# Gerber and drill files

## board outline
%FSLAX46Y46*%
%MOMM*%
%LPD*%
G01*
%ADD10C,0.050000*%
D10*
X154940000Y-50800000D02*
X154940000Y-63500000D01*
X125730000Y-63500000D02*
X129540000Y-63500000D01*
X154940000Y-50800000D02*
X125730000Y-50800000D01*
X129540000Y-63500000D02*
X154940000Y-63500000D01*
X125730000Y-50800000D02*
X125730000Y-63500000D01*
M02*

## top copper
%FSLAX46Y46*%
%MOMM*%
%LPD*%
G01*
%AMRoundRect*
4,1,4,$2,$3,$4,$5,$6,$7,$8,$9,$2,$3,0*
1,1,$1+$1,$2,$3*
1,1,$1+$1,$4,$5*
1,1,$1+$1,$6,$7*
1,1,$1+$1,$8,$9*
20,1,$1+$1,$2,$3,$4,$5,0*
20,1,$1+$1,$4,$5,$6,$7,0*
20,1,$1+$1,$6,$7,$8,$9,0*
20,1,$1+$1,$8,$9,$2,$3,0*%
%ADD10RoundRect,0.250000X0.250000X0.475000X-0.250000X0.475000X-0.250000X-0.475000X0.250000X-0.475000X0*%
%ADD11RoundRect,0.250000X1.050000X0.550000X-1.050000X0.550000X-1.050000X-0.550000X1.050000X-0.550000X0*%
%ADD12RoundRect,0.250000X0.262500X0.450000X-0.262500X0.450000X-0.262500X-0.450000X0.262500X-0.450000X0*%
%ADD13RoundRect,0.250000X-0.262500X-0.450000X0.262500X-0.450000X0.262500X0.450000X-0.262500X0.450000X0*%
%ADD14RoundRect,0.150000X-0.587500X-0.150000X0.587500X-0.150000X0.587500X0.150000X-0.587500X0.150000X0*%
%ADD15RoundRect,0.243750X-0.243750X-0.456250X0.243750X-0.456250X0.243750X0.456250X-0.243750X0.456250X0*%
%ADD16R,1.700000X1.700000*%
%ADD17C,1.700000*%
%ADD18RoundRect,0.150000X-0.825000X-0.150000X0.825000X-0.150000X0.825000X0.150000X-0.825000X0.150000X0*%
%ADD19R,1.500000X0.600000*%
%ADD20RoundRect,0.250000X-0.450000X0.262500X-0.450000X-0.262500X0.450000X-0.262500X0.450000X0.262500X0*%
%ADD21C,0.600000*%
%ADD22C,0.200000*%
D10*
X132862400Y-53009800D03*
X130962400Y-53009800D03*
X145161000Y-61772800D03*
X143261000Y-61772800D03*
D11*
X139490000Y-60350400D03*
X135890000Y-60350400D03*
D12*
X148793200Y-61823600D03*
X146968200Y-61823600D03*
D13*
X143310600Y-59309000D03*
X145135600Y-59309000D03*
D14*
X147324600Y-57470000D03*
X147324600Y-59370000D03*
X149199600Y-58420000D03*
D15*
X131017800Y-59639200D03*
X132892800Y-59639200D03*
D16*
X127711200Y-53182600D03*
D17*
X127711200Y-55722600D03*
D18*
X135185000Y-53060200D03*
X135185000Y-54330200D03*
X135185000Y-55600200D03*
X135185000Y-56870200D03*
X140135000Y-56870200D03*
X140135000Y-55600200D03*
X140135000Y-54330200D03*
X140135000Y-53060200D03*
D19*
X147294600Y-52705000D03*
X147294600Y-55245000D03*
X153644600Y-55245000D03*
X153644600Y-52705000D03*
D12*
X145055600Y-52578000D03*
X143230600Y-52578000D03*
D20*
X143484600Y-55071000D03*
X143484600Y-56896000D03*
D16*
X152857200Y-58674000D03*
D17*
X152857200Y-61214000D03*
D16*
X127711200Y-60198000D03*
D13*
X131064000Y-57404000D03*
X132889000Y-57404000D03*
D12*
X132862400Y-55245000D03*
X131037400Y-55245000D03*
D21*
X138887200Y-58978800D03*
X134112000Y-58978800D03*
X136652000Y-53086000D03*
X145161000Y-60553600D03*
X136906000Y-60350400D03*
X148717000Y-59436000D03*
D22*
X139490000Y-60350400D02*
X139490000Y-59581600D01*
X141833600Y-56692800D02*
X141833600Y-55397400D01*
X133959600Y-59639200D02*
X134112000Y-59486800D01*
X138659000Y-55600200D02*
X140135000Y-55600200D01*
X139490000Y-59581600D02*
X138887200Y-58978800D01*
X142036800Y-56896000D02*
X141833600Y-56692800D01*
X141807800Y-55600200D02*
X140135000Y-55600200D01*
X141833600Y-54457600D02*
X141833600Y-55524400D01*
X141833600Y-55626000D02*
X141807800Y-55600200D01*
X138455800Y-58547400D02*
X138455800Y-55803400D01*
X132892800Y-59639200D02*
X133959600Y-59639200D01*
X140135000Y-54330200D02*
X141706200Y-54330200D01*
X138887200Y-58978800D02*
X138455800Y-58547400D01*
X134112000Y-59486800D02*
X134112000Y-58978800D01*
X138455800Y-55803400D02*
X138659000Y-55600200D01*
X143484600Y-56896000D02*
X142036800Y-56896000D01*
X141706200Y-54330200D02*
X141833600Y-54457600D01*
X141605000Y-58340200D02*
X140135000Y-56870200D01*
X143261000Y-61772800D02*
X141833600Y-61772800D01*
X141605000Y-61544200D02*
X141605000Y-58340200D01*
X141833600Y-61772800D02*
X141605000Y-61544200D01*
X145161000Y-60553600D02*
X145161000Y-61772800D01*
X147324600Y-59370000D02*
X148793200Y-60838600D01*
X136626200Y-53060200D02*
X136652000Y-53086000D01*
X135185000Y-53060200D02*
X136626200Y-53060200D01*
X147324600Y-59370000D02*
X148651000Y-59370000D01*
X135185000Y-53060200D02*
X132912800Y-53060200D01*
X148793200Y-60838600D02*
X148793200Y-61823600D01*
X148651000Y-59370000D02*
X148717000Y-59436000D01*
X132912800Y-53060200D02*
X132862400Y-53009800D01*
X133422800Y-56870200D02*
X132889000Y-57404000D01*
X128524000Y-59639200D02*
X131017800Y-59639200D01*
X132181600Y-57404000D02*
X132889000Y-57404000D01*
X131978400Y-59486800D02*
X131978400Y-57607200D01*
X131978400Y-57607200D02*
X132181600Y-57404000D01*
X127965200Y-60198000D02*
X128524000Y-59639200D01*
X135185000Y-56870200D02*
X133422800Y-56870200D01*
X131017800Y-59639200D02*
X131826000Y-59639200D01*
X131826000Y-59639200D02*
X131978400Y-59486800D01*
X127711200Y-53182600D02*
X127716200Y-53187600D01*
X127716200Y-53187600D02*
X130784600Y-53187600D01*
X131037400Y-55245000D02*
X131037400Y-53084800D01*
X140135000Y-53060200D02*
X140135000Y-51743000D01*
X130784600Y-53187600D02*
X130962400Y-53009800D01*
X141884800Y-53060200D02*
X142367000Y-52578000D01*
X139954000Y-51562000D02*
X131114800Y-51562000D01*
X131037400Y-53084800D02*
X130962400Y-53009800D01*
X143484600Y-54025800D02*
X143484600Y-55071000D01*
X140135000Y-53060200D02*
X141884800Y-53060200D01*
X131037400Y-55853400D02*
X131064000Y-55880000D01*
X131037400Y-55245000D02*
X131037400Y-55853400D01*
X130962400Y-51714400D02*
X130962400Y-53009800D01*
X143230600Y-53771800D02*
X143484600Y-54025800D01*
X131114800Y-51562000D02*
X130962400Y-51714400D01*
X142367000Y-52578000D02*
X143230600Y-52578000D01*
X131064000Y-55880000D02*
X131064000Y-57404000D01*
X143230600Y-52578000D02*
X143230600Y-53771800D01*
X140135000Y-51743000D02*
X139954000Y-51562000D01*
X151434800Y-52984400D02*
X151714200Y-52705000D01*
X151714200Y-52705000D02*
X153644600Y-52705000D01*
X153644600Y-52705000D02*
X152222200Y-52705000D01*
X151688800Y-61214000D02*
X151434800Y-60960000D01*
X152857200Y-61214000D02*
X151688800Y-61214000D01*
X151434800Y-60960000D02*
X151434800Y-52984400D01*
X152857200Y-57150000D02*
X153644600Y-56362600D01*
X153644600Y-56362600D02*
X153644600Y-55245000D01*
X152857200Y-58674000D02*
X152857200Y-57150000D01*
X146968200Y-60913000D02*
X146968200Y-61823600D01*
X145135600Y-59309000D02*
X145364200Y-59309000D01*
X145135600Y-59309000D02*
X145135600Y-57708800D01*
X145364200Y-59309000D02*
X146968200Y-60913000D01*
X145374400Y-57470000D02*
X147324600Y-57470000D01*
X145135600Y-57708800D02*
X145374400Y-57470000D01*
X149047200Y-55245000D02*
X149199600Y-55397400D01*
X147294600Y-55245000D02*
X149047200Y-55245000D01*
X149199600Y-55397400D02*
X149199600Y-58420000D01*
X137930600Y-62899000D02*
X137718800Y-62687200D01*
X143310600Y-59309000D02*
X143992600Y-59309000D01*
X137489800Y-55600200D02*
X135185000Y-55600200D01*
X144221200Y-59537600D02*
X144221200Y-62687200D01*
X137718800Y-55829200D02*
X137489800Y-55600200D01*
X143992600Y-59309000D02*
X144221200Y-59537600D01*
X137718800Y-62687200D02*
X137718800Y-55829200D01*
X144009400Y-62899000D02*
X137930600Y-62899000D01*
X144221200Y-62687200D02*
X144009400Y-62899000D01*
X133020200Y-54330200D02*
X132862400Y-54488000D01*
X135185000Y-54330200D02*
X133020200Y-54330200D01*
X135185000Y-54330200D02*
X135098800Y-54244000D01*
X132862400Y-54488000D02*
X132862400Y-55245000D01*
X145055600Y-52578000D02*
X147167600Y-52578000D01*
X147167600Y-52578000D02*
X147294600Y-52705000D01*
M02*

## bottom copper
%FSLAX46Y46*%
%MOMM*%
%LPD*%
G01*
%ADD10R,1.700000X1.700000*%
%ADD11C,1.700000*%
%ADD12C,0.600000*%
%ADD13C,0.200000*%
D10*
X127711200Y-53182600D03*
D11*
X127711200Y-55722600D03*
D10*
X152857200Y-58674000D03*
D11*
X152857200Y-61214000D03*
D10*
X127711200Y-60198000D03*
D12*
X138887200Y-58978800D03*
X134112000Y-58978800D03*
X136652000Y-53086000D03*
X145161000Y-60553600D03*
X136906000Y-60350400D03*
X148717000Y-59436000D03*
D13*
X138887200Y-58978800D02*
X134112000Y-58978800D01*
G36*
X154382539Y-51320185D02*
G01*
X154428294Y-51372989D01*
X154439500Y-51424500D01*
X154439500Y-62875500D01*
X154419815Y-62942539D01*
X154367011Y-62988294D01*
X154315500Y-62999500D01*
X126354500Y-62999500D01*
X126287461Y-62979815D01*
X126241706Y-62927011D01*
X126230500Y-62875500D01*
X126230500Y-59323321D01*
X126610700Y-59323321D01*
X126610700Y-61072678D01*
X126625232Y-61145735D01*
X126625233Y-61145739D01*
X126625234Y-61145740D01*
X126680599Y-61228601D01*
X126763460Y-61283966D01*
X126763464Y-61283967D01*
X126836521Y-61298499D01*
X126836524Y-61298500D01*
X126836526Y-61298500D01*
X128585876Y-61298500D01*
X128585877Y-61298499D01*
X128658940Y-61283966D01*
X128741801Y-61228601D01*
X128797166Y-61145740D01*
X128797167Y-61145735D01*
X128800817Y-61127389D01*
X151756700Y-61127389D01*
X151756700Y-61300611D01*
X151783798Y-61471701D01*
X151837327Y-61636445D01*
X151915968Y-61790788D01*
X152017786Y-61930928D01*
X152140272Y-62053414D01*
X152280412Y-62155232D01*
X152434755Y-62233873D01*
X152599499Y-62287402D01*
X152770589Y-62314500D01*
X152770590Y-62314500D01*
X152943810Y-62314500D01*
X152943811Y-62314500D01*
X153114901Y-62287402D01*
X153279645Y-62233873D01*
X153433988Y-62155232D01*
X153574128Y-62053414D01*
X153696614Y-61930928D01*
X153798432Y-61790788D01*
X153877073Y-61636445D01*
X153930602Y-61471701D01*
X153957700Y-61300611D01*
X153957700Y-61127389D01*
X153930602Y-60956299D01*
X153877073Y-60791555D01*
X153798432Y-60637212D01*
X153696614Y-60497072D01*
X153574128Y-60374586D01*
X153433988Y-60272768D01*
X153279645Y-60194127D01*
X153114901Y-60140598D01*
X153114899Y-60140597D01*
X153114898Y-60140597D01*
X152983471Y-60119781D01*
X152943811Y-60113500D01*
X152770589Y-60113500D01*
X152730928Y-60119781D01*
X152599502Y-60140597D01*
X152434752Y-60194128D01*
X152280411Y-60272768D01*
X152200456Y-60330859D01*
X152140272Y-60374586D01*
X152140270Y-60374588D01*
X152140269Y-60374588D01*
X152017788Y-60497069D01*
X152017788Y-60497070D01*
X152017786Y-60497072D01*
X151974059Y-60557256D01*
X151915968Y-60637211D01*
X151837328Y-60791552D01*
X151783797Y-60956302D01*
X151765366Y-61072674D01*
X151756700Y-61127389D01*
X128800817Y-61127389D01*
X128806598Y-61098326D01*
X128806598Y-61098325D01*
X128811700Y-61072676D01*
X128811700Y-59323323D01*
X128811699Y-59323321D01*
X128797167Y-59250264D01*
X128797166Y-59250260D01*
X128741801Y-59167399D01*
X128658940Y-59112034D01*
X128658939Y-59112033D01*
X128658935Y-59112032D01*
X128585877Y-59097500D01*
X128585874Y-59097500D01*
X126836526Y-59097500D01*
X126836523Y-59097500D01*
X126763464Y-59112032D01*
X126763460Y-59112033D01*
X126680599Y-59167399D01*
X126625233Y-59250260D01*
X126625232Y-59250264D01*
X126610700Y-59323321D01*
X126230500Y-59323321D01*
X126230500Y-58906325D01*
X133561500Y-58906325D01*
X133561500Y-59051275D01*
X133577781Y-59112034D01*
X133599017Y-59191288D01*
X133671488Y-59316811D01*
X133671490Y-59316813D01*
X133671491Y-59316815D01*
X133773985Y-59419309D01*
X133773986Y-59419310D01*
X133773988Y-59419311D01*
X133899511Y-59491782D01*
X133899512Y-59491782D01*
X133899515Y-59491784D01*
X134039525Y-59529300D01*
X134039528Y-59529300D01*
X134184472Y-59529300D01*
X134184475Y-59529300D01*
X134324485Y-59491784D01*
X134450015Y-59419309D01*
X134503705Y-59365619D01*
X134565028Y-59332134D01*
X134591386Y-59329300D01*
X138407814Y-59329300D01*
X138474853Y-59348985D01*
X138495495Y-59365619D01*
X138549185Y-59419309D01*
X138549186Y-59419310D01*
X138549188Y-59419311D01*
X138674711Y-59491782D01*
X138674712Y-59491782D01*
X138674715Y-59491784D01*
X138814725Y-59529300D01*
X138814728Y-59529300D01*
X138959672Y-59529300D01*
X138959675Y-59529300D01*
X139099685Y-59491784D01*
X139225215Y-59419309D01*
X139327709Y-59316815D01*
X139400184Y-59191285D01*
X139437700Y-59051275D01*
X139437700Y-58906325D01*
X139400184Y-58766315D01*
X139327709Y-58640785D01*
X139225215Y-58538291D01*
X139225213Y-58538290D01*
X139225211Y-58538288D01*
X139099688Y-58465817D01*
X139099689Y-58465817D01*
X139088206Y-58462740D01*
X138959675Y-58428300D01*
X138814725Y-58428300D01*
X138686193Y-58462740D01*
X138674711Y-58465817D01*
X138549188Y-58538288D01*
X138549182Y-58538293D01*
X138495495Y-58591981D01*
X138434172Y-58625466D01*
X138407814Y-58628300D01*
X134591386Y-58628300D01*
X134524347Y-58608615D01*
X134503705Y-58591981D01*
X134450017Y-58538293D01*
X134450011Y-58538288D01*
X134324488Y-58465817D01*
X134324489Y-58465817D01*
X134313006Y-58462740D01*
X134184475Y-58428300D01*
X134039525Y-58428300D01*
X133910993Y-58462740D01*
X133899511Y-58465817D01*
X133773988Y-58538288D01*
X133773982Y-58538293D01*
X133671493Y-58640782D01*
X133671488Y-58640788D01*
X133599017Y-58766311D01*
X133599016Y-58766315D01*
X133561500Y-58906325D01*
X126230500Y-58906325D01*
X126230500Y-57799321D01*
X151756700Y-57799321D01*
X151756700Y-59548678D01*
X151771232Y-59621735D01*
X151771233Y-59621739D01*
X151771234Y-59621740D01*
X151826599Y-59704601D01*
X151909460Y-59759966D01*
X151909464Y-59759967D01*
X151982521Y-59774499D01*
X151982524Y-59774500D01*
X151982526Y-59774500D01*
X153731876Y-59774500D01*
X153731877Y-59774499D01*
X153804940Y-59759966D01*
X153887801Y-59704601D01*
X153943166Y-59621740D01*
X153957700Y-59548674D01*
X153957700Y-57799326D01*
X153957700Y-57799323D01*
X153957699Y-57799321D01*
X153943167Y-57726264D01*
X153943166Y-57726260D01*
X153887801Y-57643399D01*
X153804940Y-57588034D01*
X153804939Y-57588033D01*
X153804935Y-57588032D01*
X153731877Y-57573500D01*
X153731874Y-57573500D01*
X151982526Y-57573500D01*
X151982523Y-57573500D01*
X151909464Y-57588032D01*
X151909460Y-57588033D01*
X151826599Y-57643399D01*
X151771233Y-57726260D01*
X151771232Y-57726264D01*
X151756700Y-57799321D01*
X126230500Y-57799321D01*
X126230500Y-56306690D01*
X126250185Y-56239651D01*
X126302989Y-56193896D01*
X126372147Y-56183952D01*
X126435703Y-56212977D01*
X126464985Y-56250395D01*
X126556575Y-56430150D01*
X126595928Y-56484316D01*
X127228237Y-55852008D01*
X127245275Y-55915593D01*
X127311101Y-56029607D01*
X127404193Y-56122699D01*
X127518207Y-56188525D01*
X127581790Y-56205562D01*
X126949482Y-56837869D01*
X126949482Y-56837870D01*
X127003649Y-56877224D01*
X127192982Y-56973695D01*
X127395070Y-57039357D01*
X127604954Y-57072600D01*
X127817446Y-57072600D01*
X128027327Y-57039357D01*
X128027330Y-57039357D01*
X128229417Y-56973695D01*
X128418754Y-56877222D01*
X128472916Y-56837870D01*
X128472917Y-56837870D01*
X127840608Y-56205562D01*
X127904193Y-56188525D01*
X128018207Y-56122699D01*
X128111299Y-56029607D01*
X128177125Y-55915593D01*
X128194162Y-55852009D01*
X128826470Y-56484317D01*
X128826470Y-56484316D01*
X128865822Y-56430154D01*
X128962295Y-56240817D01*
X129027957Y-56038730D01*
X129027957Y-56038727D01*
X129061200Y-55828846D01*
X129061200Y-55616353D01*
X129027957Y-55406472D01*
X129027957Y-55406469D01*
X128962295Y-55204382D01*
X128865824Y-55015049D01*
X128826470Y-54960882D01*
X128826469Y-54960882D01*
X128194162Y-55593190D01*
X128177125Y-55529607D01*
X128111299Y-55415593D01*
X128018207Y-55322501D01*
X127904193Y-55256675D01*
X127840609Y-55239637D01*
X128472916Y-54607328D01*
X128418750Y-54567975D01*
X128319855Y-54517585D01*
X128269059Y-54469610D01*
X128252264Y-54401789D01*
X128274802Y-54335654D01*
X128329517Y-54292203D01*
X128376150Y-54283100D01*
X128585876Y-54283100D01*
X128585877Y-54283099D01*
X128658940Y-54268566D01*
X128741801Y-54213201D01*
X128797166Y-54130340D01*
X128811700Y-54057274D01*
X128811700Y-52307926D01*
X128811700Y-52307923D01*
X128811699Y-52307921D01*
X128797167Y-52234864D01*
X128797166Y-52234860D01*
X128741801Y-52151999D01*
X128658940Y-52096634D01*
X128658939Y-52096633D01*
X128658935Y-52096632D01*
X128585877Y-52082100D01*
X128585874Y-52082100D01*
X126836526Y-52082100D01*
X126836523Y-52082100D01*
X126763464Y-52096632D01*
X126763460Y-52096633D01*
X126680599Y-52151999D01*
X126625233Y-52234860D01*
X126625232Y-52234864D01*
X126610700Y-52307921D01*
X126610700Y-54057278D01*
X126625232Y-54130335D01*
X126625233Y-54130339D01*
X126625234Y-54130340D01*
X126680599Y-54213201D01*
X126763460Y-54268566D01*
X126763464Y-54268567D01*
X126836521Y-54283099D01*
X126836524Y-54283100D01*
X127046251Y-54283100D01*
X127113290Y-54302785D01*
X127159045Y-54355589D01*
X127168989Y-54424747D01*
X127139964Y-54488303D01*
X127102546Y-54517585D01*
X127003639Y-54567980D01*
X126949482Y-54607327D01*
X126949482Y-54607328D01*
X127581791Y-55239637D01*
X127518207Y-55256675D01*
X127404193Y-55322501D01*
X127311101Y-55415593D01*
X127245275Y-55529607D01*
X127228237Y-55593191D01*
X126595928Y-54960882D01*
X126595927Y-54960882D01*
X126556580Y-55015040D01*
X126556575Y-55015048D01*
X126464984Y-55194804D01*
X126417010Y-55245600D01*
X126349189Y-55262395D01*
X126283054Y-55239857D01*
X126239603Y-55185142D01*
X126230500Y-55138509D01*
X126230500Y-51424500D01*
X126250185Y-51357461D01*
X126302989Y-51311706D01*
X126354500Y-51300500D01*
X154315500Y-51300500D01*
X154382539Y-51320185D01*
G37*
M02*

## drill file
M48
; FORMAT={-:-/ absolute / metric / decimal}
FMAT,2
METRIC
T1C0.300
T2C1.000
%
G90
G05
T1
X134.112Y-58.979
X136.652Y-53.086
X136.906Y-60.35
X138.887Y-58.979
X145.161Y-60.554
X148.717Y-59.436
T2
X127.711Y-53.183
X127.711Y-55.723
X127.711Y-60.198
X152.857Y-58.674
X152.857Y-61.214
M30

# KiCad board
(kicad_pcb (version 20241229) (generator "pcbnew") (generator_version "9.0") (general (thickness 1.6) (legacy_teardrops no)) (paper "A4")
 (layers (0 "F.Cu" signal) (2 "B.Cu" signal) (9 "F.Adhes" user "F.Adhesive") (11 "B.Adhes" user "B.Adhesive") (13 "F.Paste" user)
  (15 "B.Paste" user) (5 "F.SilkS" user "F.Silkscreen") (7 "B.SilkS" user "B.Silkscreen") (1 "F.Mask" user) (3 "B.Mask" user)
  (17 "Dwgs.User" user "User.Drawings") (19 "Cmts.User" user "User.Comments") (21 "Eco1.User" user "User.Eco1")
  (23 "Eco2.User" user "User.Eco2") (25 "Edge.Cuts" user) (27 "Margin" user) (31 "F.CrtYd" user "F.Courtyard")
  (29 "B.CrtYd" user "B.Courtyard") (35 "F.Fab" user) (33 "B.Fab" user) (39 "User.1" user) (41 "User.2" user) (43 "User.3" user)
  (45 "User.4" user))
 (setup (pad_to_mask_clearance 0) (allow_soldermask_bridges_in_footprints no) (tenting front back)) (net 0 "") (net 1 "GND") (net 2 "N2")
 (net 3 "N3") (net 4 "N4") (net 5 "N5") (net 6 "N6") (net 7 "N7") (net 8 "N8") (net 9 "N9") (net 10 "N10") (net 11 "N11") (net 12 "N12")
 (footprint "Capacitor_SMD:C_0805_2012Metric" (layer "F.Cu") (at 131.9124 53.0098 180)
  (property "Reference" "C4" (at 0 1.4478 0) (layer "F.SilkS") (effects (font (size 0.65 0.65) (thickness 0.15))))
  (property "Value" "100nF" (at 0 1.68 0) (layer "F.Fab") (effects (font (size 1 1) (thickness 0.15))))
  (pad "1" smd roundrect (at -0.95 0 180) (size 1 1.45) (layers "F.Cu" "F.Mask" "F.Paste") (roundrect_rratio 0.25) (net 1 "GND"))
  (pad "2" smd roundrect (at 0.95 0 180) (size 1 1.45) (layers "F.Cu" "F.Mask" "F.Paste") (roundrect_rratio 0.25) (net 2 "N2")))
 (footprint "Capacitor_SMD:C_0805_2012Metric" (layer "F.Cu") (at 144.211 61.7728 180)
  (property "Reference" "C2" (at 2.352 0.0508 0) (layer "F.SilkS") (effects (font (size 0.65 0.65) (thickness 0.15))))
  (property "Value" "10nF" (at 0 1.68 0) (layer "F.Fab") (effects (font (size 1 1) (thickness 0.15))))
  (pad "1" smd roundrect (at -0.95 0 180) (size 1 1.45) (layers "F.Cu" "F.Mask" "F.Paste") (roundrect_rratio 0.25) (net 1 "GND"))
  (pad "2" smd roundrect (at 0.95 0 180) (size 1 1.45) (layers "F.Cu" "F.Mask" "F.Paste") (roundrect_rratio 0.25) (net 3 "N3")))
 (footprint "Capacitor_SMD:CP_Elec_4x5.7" (layer "F.Cu") (at 137.69 60.3504 180)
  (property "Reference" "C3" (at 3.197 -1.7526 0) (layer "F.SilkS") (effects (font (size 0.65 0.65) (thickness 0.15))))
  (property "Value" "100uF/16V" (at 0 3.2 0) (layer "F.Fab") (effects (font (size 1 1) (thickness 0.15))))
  (pad "1" smd roundrect (at -1.8 0 180) (size 2.6 1.6) (layers "F.Cu" "F.Mask" "F.Paste") (roundrect_rratio 0.15625) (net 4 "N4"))
  (pad "2" smd roundrect (at 1.8 0 180) (size 2.6 1.6) (layers "F.Cu" "F.Mask" "F.Paste") (roundrect_rratio 0.15625) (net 1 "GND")))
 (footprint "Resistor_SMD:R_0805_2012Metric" (layer "F.Cu") (at 147.8807 61.8236 180)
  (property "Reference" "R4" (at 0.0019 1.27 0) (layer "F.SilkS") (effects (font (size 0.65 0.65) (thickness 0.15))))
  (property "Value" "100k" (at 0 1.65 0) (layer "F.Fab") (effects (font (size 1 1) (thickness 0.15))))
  (pad "1" smd roundrect (at -0.9125 0 180) (size 1.025 1.4) (layers "F.Cu" "F.Mask" "F.Paste") (roundrect_rratio 0.243902) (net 1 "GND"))
  (pad "2" smd roundrect (at 0.9125 0 180) (size 1.025 1.4) (layers "F.Cu" "F.Mask" "F.Paste") (roundrect_rratio 0.243902) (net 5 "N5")))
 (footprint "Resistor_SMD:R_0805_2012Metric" (layer "F.Cu") (at 144.2231 59.309)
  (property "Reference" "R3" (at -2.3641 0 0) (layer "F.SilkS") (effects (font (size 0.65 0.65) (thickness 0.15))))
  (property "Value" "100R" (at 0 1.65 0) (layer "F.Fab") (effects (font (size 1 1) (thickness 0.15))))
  (pad "1" smd roundrect (at -0.9125 0) (size 1.025 1.4) (layers "F.Cu" "F.Mask" "F.Paste") (roundrect_rratio 0.243902) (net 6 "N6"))
  (pad "2" smd roundrect (at 0.9125 0) (size 1.025 1.4) (layers "F.Cu" "F.Mask" "F.Paste") (roundrect_rratio 0.243902) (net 5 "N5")))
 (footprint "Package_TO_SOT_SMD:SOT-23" (layer "F.Cu") (at 148.2621 58.42)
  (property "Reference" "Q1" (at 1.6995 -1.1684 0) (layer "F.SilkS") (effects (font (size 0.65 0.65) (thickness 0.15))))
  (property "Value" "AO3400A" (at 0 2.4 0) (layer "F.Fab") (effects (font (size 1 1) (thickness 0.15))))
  (pad "1" smd roundrect (at -0.9375 -0.95) (size 1.475 0.6) (layers "F.Cu" "F.Mask" "F.Paste") (roundrect_rratio 0.25) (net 5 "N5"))
  (pad "2" smd roundrect (at -0.9375 0.95) (size 1.475 0.6) (layers "F.Cu" "F.Mask" "F.Paste") (roundrect_rratio 0.25) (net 1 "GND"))
  (pad "3" smd roundrect (at 0.9375 0) (size 1.475 0.6) (layers "F.Cu" "F.Mask" "F.Paste") (roundrect_rratio 0.25) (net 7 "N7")))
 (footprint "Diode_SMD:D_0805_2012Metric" (layer "F.Cu") (at 131.9553 59.6392)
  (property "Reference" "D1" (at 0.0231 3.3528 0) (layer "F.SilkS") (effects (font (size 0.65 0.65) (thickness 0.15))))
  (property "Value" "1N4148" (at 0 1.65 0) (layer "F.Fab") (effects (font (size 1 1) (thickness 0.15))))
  (pad "1" smd roundrect (at -0.9375 0) (size 0.975 1.4) (layers "F.Cu" "F.Mask" "F.Paste") (roundrect_rratio 0.25) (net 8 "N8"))
  (pad "2" smd roundrect (at 0.9375 0) (size 0.975 1.4) (layers "F.Cu" "F.Mask" "F.Paste") (roundrect_rratio 0.25) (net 4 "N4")))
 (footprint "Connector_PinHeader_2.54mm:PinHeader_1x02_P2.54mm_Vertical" (layer "F.Cu") (at 127.7112 53.1826)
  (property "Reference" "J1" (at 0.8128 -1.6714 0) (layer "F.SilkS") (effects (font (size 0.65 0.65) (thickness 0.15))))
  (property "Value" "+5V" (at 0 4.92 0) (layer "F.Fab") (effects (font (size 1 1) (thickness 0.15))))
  (pad "1" thru_hole rect (at 0 0) (size 1.7 1.7) (drill 1) (layers "*.Cu" "*.Mask") (remove_unused_layers no) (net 2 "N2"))
  (pad "2" thru_hole circle (at 0 2.54) (size 1.7 1.7) (drill 1) (layers "*.Cu" "*.Mask") (remove_unused_layers no) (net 1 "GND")))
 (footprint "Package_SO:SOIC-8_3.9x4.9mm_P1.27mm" (layer "F.Cu") (at 137.66 54.9652)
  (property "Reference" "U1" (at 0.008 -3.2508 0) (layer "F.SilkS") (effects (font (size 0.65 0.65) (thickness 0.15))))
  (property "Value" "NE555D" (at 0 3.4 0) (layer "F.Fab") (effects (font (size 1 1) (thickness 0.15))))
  (pad "1" smd roundrect (at -2.475 -1.905) (size 1.95 0.6) (layers "F.Cu" "F.Mask" "F.Paste") (roundrect_rratio 0.25) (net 1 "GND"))
  (pad "2" smd roundrect (at -2.475 -0.635) (size 1.95 0.6) (layers "F.Cu" "F.Mask" "F.Paste") (roundrect_rratio 0.25) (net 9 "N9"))
  (pad "3" smd roundrect (at -2.475 0.635) (size 1.95 0.6) (layers "F.Cu" "F.Mask" "F.Paste") (roundrect_rratio 0.25) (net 6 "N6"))
  (pad "4" smd roundrect (at -2.475 1.905) (size 1.95 0.6) (layers "F.Cu" "F.Mask" "F.Paste") (roundrect_rratio 0.25) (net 8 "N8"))
  (pad "5" smd roundrect (at 2.475 1.905) (size 1.95 0.6) (layers "F.Cu" "F.Mask" "F.Paste") (roundrect_rratio 0.25) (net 3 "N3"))
  (pad "6" smd roundrect (at 2.475 0.635) (size 1.95 0.6) (layers "F.Cu" "F.Mask" "F.Paste") (roundrect_rratio 0.25) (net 4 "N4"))
  (pad "7" smd roundrect (at 2.475 -0.635) (size 1.95 0.6) (layers "F.Cu" "F.Mask" "F.Paste") (roundrect_rratio 0.25) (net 4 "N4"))
  (pad "8" smd roundrect (at 2.475 -1.905) (size 1.95 0.6) (layers "F.Cu" "F.Mask" "F.Paste") (roundrect_rratio 0.25) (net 2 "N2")))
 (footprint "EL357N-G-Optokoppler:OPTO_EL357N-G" (layer "F.Cu") (at 150.4696 53.975)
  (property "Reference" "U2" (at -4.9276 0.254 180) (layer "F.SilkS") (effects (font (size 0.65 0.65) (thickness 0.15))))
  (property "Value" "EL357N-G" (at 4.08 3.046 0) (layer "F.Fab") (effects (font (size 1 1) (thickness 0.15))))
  (pad "1" smd rect (at -3.175 -1.27) (size 1.5 0.6) (layers "F.Cu" "F.Mask" "F.Paste") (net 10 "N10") (solder_mask_margin 0.102))
  (pad "2" smd rect (at -3.175 1.27) (size 1.5 0.6) (layers "F.Cu" "F.Mask" "F.Paste") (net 7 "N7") (solder_mask_margin 0.102))
  (pad "3" smd rect (at 3.175 1.27) (size 1.5 0.6) (layers "F.Cu" "F.Mask" "F.Paste") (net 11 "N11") (solder_mask_margin 0.102))
  (pad "4" smd rect (at 3.175 -1.27) (size 1.5 0.6) (layers "F.Cu" "F.Mask" "F.Paste") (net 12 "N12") (solder_mask_margin 0.102)))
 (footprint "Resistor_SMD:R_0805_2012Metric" (layer "F.Cu") (at 144.1431 52.578 180)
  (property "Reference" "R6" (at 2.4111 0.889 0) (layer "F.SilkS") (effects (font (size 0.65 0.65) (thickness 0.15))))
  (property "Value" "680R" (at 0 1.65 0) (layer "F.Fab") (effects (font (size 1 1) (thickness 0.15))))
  (pad "1" smd roundrect (at -0.9125 0 180) (size 1.025 1.4) (layers "F.Cu" "F.Mask" "F.Paste") (roundrect_rratio 0.243902) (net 10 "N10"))
  (pad "2" smd roundrect (at 0.9125 0 180) (size 1.025 1.4) (layers "F.Cu" "F.Mask" "F.Paste") (roundrect_rratio 0.243902) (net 2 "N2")))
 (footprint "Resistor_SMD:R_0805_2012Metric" (layer "F.Cu") (at 143.4846 55.9835 -90)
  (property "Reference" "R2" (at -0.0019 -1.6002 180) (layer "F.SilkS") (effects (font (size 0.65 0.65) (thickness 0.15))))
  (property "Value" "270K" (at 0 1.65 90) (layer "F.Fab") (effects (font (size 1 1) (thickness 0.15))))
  (pad "1" smd roundrect (at -0.9125 0 270) (size 1.025 1.4) (layers "F.Cu" "F.Mask" "F.Paste") (roundrect_rratio 0.243902) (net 2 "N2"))
  (pad "2" smd roundrect (at 0.9125 0 270) (size 1.025 1.4) (layers "F.Cu" "F.Mask" "F.Paste") (roundrect_rratio 0.243902) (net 4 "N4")))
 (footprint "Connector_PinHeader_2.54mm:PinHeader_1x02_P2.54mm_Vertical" (layer "F.Cu") (at 152.8572 58.674)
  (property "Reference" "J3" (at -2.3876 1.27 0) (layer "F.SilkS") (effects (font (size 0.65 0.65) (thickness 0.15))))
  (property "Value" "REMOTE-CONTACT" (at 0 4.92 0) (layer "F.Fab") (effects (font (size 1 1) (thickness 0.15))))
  (pad "1" thru_hole rect (at 0 0) (size 1.7 1.7) (drill 1) (layers "*.Cu" "*.Mask") (remove_unused_layers no) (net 11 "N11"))
  (pad "2" thru_hole circle (at 0 2.54) (size 1.7 1.7) (drill 1) (layers "*.Cu" "*.Mask") (remove_unused_layers no) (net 12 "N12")))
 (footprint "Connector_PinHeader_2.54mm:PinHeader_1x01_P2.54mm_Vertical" (layer "F.Cu") (at 127.7112 60.198)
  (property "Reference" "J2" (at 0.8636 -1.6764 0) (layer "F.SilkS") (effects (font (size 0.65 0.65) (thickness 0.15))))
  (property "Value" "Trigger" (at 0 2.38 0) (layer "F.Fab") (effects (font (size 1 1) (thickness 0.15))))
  (pad "1" thru_hole rect (at 0 0) (size 1.7 1.7) (drill 1) (layers "*.Cu" "*.Mask") (remove_unused_layers no) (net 8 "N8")))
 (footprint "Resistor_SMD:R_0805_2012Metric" (layer "F.Cu") (at 131.9765 57.404)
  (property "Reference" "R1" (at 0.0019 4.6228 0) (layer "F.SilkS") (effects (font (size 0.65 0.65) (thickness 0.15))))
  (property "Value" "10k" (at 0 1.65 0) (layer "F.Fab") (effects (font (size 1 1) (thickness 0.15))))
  (pad "1" smd roundrect (at -0.9125 0) (size 1.025 1.4) (layers "F.Cu" "F.Mask" "F.Paste") (roundrect_rratio 0.243902) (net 2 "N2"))
  (pad "2" smd roundrect (at 0.9125 0) (size 1.025 1.4) (layers "F.Cu" "F.Mask" "F.Paste") (roundrect_rratio 0.243902) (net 8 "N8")))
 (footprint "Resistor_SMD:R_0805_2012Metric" (layer "F.Cu") (at 131.9499 55.245 180)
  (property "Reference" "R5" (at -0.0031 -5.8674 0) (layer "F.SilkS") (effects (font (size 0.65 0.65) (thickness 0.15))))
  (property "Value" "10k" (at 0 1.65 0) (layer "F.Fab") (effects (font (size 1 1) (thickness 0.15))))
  (pad "1" smd roundrect (at -0.9125 0 180) (size 1.025 1.4) (layers "F.Cu" "F.Mask" "F.Paste") (roundrect_rratio 0.243902) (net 9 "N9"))
  (pad "2" smd roundrect (at 0.9125 0 180) (size 1.025 1.4) (layers "F.Cu" "F.Mask" "F.Paste") (roundrect_rratio 0.243902) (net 2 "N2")))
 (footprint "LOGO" (layer "B.Cu") (at 140.84617 57.489081 180)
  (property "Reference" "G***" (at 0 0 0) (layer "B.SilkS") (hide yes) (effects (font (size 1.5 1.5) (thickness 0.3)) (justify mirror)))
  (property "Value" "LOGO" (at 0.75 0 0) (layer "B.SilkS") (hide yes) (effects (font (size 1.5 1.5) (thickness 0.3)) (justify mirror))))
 (gr_line (start 154.94 50.8) (end 154.94 63.5) (stroke (width 0.05) (type default)) (layer "Edge.Cuts"))
 (gr_line (start 125.73 63.5) (end 129.54 63.5) (stroke (width 0.05) (type default)) (layer "Edge.Cuts"))
 (gr_line (start 154.94 50.8) (end 125.73 50.8) (stroke (width 0.05) (type default)) (layer "Edge.Cuts"))
 (gr_line (start 129.54 63.5) (end 154.94 63.5) (stroke (width 0.05) (type default)) (layer "Edge.Cuts"))
 (gr_line (start 125.73 50.8) (end 125.73 63.5) (stroke (width 0.05) (type default)) (layer "Edge.Cuts"))
 (segment (start 139.49 60.3504) (end 139.49 59.5816) (width 0.2) (layer "F.Cu") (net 4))
 (segment (start 141.8336 56.6928) (end 141.8336 55.3974) (width 0.2) (layer "F.Cu") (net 4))
 (segment (start 133.9596 59.6392) (end 134.112 59.4868) (width 0.2) (layer "F.Cu") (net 4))
 (segment (start 138.659 55.6002) (end 140.135 55.6002) (width 0.2) (layer "F.Cu") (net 4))
 (segment (start 139.49 59.5816) (end 138.8872 58.9788) (width 0.2) (layer "F.Cu") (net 4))
 (segment (start 142.0368 56.896) (end 141.8336 56.6928) (width 0.2) (layer "F.Cu") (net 4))
 (segment (start 141.8078 55.6002) (end 140.135 55.6002) (width 0.2) (layer "F.Cu") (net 4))
 (segment (start 141.8336 54.4576) (end 141.8336 55.5244) (width 0.2) (layer "F.Cu") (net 4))
 (segment (start 141.8336 55.626) (end 141.8078 55.6002) (width 0.2) (layer "F.Cu") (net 4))
 (segment (start 138.4558 58.5474) (end 138.4558 55.8034) (width 0.2) (layer "F.Cu") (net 4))
 (segment (start 132.8928 59.6392) (end 133.9596 59.6392) (width 0.2) (layer "F.Cu") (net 4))
 (segment (start 140.135 54.3302) (end 141.7062 54.3302) (width 0.2) (layer "F.Cu") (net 4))
 (segment (start 138.8872 58.9788) (end 138.4558 58.5474) (width 0.2) (layer "F.Cu") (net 4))
 (segment (start 134.112 59.4868) (end 134.112 58.9788) (width 0.2) (layer "F.Cu") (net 4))
 (segment (start 138.4558 55.8034) (end 138.659 55.6002) (width 0.2) (layer "F.Cu") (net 4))
 (segment (start 143.4846 56.896) (end 142.0368 56.896) (width 0.2) (layer "F.Cu") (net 4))
 (segment (start 141.7062 54.3302) (end 141.8336 54.4576) (width 0.2) (layer "F.Cu") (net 4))
 (via (at 138.8872 58.9788) (size 0.6) (drill 0.3) (layers "F.Cu" "B.Cu") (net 4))
 (via (at 134.112 58.9788) (size 0.6) (drill 0.3) (layers "F.Cu" "B.Cu") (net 4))
 (segment (start 138.8872 58.9788) (end 134.112 58.9788) (width 0.2) (layer "B.Cu") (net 4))
 (segment (start 141.605 58.3402) (end 140.135 56.8702) (width 0.2) (layer "F.Cu") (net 3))
 (segment (start 143.261 61.7728) (end 141.8336 61.7728) (width 0.2) (layer "F.Cu") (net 3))
 (segment (start 141.605 61.5442) (end 141.605 58.3402) (width 0.2) (layer "F.Cu") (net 3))
 (segment (start 141.8336 61.7728) (end 141.605 61.5442) (width 0.2) (layer "F.Cu") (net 3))
 (segment (start 145.161 60.5536) (end 145.161 61.7728) (width 0.2) (layer "F.Cu") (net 1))
 (segment (start 147.3246 59.37) (end 148.7932 60.8386) (width 0.2) (layer "F.Cu") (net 1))
 (segment (start 136.6262 53.0602) (end 136.652 53.086) (width 0.2) (layer "F.Cu") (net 1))
 (segment (start 135.185 53.0602) (end 136.6262 53.0602) (width 0.2) (layer "F.Cu") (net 1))
 (segment (start 147.3246 59.37) (end 148.651 59.37) (width 0.2) (layer "F.Cu") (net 1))
 (segment (start 135.185 53.0602) (end 132.9128 53.0602) (width 0.2) (layer "F.Cu") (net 1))
 (segment (start 148.7932 60.8386) (end 148.7932 61.8236) (width 0.2) (layer "F.Cu") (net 1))
 (segment (start 148.651 59.37) (end 148.717 59.436) (width 0.2) (layer "F.Cu") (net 1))
 (segment (start 132.9128 53.0602) (end 132.8624 53.0098) (width 0.2) (layer "F.Cu") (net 1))
 (via (at 136.652 53.086) (size 0.6) (drill 0.3) (layers "F.Cu" "B.Cu") (free yes) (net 1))
 (via (at 145.161 60.5536) (size 0.6) (drill 0.3) (layers "F.Cu" "B.Cu") (free yes) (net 1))
 (via (at 136.906 60.3504) (size 0.6) (drill 0.3) (layers "F.Cu" "B.Cu") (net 1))
 (via (at 148.717 59.436) (size 0.6) (drill 0.3) (layers "F.Cu" "B.Cu") (free yes) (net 1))
 (segment (start 133.4228 56.8702) (end 132.889 57.404) (width 0.2) (layer "F.Cu") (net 8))
 (segment (start 128.524 59.6392) (end 131.0178 59.6392) (width 0.2) (layer "F.Cu") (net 8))
 (segment (start 132.1816 57.404) (end 132.889 57.404) (width 0.2) (layer "F.Cu") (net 8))
 (segment (start 131.9784 59.4868) (end 131.9784 57.6072) (width 0.2) (layer "F.Cu") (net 8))
 (segment (start 131.9784 57.6072) (end 132.1816 57.404) (width 0.2) (layer "F.Cu") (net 8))
 (segment (start 127.9652 60.198) (end 128.524 59.6392) (width 0.2) (layer "F.Cu") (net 8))
 (segment (start 135.185 56.8702) (end 133.4228 56.8702) (width 0.2) (layer "F.Cu") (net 8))
 (segment (start 131.0178 59.6392) (end 131.826 59.6392) (width 0.2) (layer "F.Cu") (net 8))
 (segment (start 131.826 59.6392) (end 131.9784 59.4868) (width 0.2) (layer "F.Cu") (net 8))
 (segment (start 127.7112 53.1826) (end 127.7162 53.1876) (width 0.2) (layer "F.Cu") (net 2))
 (segment (start 127.7162 53.1876) (end 130.7846 53.1876) (width 0.2) (layer "F.Cu") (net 2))
 (segment (start 131.0374 55.245) (end 131.0374 53.0848) (width 0.2) (layer "F.Cu") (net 2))
 (segment (start 140.135 53.0602) (end 140.135 51.743) (width 0.2) (layer "F.Cu") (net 2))
 (segment (start 130.7846 53.1876) (end 130.9624 53.0098) (width 0.2) (layer "F.Cu") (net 2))
 (segment (start 141.8848 53.0602) (end 142.367 52.578) (width 0.2) (layer "F.Cu") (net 2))
 (segment (start 139.954 51.562) (end 131.1148 51.562) (width 0.2) (layer "F.Cu") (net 2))
 (segment (start 131.0374 53.0848) (end 130.9624 53.0098) (width 0.2) (layer "F.Cu") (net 2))
 (segment (start 143.4846 54.0258) (end 143.4846 55.071) (width 0.2) (layer "F.Cu") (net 2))
 (segment (start 140.135 53.0602) (end 141.8848 53.0602) (width 0.2) (layer "F.Cu") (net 2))
 (segment (start 131.0374 55.8534) (end 131.064 55.88) (width 0.2) (layer "F.Cu") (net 2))
 (segment (start 131.0374 55.245) (end 131.0374 55.8534) (width 0.2) (layer "F.Cu") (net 2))
 (segment (start 130.9624 51.7144) (end 130.9624 53.0098) (width 0.2) (layer "F.Cu") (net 2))
 (segment (start 143.2306 53.7718) (end 143.4846 54.0258) (width 0.2) (layer "F.Cu") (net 2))
 (segment (start 131.1148 51.562) (end 130.9624 51.7144) (width 0.2) (layer "F.Cu") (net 2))
 (segment (start 142.367 52.578) (end 143.2306 52.578) (width 0.2) (layer "F.Cu") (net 2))
 (segment (start 131.064 55.88) (end 131.064 57.404) (width 0.2) (layer "F.Cu") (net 2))
 (segment (start 143.2306 52.578) (end 143.2306 53.7718) (width 0.2) (layer "F.Cu") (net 2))
 (segment (start 140.135 51.743) (end 139.954 51.562) (width 0.2) (layer "F.Cu") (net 2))
 (segment (start 151.4348 52.9844) (end 151.7142 52.705) (width 0.2) (layer "F.Cu") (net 12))
 (segment (start 151.7142 52.705) (end 153.6446 52.705) (width 0.2) (layer "F.Cu") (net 12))
 (segment (start 153.6446 52.705) (end 152.2222 52.705) (width 0.2) (layer "F.Cu") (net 12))
 (segment (start 151.6888 61.214) (end 151.4348 60.96) (width 0.2) (layer "F.Cu") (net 12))
 (segment (start 152.8572 61.214) (end 151.6888 61.214) (width 0.2) (layer "F.Cu") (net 12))
 (segment (start 151.4348 60.96) (end 151.4348 52.9844) (width 0.2) (layer "F.Cu") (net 12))
 (segment (start 152.8572 57.15) (end 153.6446 56.3626) (width 0.2) (layer "F.Cu") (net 11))
 (segment (start 153.6446 56.3626) (end 153.6446 55.245) (width 0.2) (layer "F.Cu") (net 11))
 (segment (start 152.8572 58.674) (end 152.8572 57.15) (width 0.2) (layer "F.Cu") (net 11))
 (segment (start 146.9682 60.913) (end 146.9682 61.8236) (width 0.2) (layer "F.Cu") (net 5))
 (segment (start 145.1356 59.309) (end 145.3642 59.309) (width 0.2) (layer "F.Cu") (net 5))
 (segment (start 145.1356 59.309) (end 145.1356 57.7088) (width 0.2) (layer "F.Cu") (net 5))
 (segment (start 145.3642 59.309) (end 146.9682 60.913) (width 0.2) (layer "F.Cu") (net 5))
 (segment (start 145.3744 57.47) (end 147.3246 57.47) (width 0.2) (layer "F.Cu") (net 5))
 (segment (start 145.1356 57.7088) (end 145.3744 57.47) (width 0.2) (layer "F.Cu") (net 5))
 (segment (start 149.0472 55.245) (end 149.1996 55.3974) (width 0.2) (layer "F.Cu") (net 7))
 (segment (start 147.2946 55.245) (end 149.0472 55.245) (width 0.2) (layer "F.Cu") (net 7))
 (segment (start 149.1996 55.3974) (end 149.1996 58.42) (width 0.2) (layer "F.Cu") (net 7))
 (segment (start 137.9306 62.899) (end 137.7188 62.6872) (width 0.2) (layer "F.Cu") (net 6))
 (segment (start 143.3106 59.309) (end 143.9926 59.309) (width 0.2) (layer "F.Cu") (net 6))
 (segment (start 137.4898 55.6002) (end 135.185 55.6002) (width 0.2) (layer "F.Cu") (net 6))
 (segment (start 144.2212 59.5376) (end 144.2212 62.6872) (width 0.2) (layer "F.Cu") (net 6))
 (segment (start 137.7188 55.8292) (end 137.4898 55.6002) (width 0.2) (layer "F.Cu") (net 6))
 (segment (start 143.9926 59.309) (end 144.2212 59.5376) (width 0.2) (layer "F.Cu") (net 6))
 (segment (start 137.7188 62.6872) (end 137.7188 55.8292) (width 0.2) (layer "F.Cu") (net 6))
 (segment (start 144.0094 62.899) (end 137.9306 62.899) (width 0.2) (layer "F.Cu") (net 6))
 (segment (start 144.2212 62.6872) (end 144.0094 62.899) (width 0.2) (layer "F.Cu") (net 6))
 (segment (start 133.0202 54.3302) (end 132.8624 54.488) (width 0.2) (layer "F.Cu") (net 9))
 (segment (start 135.185 54.3302) (end 133.0202 54.3302) (width 0.2) (layer "F.Cu") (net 9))
 (segment (start 135.185 54.3302) (end 135.0988 54.244) (width 0.2) (layer "F.Cu") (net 9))
 (segment (start 132.8624 54.488) (end 132.8624 55.245) (width 0.2) (layer "F.Cu") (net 9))
 (segment (start 145.0556 52.578) (end 147.1676 52.578) (width 0.2) (layer "F.Cu") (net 10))
 (segment (start 147.1676 52.578) (end 147.2946 52.705) (width 0.2) (layer "F.Cu") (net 10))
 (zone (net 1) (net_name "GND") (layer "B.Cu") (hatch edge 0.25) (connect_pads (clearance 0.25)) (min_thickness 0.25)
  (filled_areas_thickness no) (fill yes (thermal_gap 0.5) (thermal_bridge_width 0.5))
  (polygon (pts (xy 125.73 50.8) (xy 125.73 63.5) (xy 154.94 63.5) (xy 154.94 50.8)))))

